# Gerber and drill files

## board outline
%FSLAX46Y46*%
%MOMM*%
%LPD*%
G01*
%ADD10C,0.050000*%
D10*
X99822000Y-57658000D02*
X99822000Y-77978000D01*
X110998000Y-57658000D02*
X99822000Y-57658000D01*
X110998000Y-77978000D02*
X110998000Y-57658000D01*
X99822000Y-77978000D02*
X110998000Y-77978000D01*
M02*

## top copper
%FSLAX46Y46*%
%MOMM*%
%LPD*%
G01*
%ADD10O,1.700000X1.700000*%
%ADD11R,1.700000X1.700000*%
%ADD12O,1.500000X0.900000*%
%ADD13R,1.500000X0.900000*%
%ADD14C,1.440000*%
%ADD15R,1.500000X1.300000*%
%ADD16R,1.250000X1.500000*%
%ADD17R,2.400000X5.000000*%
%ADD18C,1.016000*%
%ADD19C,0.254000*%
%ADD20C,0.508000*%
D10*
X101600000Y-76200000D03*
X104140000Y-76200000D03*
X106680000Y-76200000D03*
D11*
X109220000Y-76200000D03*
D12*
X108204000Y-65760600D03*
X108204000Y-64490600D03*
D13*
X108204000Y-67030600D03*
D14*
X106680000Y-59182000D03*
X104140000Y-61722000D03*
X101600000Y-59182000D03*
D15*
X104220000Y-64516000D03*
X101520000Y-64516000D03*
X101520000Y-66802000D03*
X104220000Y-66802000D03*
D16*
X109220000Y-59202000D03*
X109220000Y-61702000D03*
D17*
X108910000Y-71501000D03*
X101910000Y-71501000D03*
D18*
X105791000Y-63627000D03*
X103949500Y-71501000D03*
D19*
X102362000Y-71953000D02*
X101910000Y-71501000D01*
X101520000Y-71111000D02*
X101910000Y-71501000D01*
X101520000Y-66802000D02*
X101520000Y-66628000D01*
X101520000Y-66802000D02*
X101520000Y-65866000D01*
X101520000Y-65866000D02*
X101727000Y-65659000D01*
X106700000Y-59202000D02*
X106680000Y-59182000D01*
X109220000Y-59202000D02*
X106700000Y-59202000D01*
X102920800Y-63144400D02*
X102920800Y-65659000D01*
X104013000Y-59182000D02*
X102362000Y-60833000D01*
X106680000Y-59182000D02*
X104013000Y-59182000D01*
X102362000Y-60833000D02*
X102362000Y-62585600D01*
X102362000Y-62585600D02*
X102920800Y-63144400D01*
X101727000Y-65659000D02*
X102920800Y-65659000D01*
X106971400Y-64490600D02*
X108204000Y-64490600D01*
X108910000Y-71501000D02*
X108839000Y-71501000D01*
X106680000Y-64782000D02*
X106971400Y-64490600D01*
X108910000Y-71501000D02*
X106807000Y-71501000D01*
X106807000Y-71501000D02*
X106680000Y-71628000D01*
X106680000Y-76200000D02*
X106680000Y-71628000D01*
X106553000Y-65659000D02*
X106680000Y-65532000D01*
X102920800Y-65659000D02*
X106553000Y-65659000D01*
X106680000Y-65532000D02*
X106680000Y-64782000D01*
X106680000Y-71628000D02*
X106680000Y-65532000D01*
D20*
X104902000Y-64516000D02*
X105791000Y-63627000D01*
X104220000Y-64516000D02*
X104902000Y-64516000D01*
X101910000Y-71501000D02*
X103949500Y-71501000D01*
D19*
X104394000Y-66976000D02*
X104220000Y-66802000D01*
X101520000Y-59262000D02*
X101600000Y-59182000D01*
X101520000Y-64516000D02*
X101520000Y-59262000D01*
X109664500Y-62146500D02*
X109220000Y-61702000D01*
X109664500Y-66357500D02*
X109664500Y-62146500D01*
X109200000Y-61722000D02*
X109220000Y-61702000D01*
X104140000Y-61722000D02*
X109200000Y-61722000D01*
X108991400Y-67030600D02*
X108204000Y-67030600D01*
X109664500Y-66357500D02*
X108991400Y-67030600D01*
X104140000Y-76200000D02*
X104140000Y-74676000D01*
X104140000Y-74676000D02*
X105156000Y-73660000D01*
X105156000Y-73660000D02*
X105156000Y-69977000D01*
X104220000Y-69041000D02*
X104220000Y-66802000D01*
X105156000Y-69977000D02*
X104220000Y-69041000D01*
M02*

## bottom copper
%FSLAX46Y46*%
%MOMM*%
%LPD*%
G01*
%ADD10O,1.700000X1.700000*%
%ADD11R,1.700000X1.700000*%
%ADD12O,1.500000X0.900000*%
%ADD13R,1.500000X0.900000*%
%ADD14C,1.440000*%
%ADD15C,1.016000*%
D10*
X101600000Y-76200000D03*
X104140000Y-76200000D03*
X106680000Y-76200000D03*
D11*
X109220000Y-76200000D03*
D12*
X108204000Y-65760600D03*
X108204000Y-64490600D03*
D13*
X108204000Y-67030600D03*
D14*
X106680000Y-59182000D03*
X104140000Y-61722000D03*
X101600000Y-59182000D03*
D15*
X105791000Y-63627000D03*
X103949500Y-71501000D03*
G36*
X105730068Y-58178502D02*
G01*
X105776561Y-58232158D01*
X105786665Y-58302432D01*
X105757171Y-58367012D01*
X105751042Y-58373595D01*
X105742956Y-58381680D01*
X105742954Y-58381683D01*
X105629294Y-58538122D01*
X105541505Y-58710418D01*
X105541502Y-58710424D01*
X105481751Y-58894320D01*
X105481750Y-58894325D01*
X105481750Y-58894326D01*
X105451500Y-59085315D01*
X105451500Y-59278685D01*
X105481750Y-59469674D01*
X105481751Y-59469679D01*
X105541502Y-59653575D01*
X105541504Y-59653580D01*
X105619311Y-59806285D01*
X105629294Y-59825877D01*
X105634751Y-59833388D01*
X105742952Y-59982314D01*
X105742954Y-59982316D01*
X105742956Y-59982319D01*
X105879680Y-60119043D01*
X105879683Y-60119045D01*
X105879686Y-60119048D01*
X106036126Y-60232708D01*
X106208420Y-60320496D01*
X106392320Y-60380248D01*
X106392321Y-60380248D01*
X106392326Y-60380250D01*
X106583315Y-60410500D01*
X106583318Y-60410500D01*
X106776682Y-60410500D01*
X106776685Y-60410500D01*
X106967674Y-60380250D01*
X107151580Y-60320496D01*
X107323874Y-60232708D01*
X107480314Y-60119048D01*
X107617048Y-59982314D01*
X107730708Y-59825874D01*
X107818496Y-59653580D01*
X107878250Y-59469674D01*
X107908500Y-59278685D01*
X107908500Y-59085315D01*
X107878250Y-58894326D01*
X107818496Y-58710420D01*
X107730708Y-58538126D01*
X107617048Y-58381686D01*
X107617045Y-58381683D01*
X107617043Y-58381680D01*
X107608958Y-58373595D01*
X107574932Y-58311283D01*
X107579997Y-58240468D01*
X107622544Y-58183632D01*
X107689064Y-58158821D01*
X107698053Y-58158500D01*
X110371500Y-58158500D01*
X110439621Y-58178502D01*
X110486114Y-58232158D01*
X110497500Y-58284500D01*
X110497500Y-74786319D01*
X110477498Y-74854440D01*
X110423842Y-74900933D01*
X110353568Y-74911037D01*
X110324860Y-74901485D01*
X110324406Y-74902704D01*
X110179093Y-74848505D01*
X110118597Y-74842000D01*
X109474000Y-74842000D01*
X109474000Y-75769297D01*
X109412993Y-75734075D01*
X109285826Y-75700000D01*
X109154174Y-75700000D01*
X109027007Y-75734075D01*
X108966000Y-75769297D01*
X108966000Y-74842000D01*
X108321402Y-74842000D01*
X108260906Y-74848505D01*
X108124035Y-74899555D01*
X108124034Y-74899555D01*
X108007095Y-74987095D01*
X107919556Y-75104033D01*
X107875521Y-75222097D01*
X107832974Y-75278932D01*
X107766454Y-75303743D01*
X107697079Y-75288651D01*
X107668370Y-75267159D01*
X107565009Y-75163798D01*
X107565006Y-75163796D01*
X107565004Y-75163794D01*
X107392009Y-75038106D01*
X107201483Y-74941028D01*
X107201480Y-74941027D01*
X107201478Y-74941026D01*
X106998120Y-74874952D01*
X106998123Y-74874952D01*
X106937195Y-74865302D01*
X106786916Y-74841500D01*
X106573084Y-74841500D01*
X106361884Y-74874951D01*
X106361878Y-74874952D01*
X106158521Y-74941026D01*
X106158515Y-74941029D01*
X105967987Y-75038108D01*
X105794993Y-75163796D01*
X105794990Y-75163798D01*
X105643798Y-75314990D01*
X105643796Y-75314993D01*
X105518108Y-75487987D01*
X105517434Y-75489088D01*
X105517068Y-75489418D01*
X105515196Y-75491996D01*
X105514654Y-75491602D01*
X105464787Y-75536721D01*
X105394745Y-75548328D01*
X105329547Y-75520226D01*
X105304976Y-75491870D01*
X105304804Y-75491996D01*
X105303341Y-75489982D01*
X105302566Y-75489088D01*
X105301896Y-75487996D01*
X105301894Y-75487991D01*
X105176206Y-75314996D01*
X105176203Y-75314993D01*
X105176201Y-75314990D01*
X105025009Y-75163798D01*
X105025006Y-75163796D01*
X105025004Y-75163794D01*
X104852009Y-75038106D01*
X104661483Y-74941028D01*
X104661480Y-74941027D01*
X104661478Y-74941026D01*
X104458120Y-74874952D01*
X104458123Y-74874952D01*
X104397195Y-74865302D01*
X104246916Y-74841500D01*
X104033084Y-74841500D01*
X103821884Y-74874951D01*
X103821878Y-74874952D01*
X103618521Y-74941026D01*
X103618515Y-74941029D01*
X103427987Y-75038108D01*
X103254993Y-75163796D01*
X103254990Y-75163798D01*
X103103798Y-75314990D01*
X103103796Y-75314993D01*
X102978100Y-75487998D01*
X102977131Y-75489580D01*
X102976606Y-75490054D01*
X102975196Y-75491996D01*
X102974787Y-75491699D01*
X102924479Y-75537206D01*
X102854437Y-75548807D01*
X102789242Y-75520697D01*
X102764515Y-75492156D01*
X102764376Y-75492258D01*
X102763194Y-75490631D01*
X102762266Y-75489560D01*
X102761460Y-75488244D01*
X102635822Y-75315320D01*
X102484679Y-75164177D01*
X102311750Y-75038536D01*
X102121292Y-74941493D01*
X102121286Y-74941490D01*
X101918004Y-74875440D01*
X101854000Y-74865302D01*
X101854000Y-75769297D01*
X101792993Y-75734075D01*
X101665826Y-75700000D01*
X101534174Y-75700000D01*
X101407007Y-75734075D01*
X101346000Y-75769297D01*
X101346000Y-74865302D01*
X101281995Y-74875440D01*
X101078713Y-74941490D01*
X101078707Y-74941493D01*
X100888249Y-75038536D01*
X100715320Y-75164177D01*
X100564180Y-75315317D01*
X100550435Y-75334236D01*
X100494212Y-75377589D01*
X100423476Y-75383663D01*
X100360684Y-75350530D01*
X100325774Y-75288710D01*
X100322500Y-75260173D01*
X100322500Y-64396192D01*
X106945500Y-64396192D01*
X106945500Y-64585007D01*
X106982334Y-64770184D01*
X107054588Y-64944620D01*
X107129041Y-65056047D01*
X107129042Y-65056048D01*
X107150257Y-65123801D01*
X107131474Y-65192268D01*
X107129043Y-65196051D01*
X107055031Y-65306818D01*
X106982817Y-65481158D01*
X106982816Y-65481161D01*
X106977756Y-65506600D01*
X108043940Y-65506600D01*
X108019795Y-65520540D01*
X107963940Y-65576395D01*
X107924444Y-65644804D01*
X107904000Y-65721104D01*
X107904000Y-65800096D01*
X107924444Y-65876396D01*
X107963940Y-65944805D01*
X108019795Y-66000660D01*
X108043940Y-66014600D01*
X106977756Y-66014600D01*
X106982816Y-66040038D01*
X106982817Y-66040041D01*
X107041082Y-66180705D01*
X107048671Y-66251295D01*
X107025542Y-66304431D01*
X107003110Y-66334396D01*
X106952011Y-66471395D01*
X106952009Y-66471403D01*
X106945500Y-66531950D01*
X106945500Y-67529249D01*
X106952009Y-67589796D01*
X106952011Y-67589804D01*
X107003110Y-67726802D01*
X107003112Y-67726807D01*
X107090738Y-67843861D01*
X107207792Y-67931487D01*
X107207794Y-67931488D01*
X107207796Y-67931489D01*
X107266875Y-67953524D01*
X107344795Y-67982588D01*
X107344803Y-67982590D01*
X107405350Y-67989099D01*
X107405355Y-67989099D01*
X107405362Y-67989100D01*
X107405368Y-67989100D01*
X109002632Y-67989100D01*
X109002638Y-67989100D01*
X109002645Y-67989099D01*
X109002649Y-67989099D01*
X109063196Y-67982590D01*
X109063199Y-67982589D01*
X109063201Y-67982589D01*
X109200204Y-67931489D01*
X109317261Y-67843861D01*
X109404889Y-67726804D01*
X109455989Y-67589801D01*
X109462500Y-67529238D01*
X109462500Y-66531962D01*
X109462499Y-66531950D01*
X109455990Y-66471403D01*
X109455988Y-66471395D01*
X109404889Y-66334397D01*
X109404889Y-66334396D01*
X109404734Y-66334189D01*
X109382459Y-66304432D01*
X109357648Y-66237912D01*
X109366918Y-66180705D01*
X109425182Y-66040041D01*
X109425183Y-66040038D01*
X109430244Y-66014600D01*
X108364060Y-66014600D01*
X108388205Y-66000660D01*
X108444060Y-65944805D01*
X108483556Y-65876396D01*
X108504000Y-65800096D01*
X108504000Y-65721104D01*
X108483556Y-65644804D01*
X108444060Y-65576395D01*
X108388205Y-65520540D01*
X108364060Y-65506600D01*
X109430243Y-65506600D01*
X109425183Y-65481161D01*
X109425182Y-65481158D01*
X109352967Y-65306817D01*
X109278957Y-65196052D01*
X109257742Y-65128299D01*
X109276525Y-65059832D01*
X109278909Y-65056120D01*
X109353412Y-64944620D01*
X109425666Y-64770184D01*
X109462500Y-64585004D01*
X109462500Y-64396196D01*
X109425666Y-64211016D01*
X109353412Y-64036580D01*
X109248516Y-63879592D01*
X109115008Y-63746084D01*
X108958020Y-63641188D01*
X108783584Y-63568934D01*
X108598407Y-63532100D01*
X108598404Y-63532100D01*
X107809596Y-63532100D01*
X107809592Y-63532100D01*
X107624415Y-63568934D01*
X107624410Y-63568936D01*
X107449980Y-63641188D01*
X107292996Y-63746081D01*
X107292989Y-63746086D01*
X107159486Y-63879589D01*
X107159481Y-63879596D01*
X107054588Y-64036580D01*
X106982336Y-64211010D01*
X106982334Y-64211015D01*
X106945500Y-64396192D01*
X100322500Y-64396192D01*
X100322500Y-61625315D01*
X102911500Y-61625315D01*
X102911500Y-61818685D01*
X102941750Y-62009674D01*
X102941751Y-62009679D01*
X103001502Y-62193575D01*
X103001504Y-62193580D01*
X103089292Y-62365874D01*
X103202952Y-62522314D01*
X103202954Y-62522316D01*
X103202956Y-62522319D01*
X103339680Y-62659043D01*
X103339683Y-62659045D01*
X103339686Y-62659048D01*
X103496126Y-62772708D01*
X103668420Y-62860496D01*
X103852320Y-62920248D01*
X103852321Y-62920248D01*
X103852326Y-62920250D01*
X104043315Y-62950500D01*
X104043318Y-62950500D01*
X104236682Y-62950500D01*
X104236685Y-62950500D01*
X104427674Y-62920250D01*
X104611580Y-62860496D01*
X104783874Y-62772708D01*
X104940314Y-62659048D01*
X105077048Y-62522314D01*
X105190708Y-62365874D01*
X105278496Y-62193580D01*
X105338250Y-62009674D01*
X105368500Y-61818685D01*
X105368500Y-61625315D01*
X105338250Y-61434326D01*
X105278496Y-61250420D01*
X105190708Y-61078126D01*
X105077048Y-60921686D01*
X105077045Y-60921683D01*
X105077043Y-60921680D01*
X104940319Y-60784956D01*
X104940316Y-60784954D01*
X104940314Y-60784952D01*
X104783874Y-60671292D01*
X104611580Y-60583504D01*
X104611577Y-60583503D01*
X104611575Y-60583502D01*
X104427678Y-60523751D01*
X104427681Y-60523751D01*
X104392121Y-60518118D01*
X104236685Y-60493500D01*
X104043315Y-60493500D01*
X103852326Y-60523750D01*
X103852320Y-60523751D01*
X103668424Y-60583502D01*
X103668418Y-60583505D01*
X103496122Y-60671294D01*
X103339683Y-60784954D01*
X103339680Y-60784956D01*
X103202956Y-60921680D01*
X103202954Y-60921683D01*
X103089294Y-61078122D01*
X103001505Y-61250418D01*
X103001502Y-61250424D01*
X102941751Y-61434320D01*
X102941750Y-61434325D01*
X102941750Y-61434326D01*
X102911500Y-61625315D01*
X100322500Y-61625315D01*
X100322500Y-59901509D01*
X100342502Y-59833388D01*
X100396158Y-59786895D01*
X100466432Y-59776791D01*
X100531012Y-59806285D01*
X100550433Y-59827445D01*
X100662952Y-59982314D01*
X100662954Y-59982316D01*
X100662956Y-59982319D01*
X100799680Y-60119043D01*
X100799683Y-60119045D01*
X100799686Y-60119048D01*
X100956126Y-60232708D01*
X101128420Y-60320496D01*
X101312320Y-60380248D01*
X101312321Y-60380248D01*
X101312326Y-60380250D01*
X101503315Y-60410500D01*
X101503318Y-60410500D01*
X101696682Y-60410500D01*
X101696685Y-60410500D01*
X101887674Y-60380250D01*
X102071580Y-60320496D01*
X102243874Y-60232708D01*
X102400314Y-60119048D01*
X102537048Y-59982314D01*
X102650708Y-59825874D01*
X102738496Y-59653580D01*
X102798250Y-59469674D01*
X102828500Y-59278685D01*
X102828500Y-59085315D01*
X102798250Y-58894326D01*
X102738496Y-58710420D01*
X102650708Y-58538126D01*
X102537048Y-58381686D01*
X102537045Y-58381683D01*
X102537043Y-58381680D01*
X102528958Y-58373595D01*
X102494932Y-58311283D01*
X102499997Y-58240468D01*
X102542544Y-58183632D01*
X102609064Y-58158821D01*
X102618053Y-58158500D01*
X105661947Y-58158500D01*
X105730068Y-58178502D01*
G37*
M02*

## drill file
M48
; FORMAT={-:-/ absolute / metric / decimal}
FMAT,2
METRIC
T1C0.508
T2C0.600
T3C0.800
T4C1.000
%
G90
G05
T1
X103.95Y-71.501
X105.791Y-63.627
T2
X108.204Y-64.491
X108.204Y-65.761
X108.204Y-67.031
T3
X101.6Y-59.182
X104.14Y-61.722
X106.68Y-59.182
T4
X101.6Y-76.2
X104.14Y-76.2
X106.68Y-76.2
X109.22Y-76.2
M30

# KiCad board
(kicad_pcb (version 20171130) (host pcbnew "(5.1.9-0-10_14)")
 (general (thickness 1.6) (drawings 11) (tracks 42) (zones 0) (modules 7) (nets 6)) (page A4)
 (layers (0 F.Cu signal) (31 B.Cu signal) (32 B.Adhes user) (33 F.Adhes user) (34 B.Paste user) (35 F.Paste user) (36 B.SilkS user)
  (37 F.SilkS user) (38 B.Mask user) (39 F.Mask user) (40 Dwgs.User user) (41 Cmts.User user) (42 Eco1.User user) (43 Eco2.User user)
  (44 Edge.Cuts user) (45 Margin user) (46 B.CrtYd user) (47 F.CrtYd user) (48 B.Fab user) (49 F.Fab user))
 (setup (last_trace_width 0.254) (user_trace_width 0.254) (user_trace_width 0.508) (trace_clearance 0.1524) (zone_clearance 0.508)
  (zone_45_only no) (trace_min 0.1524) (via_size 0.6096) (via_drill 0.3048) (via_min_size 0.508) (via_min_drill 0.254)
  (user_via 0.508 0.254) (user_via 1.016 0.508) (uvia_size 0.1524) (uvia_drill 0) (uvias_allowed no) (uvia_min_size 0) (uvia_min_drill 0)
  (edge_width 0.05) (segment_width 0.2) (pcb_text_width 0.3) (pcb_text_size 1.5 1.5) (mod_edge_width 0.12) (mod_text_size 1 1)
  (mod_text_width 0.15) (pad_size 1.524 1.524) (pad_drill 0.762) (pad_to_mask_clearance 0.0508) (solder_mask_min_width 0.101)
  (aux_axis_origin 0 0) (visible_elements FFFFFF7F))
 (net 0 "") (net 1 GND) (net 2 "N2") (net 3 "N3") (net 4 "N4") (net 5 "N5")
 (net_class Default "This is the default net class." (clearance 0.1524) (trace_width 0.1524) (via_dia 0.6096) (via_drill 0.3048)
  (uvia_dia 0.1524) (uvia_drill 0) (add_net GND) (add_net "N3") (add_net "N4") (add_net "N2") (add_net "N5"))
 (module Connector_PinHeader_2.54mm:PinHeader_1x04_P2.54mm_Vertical (layer B.Cu) (at 109.22 76.2 90)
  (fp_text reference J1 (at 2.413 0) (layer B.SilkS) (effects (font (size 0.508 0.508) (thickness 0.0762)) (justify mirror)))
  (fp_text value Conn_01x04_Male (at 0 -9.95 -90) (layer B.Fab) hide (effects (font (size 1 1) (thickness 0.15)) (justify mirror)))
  (pad 4 thru_hole oval (at 0 -7.62 90) (size 1.7 1.7) (drill 1) (layers *.Cu *.Mask) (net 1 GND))
  (pad 3 thru_hole oval (at 0 -5.08 90) (size 1.7 1.7) (drill 1) (layers *.Cu *.Mask) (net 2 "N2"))
  (pad 2 thru_hole oval (at 0 -2.54 90) (size 1.7 1.7) (drill 1) (layers *.Cu *.Mask) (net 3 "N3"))
  (pad 1 thru_hole rect (at 0 0 90) (size 1.7 1.7) (drill 1) (layers *.Cu *.Mask) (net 1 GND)))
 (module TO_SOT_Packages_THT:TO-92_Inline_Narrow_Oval (layer F.Cu) (at 108.204 67.0306 90)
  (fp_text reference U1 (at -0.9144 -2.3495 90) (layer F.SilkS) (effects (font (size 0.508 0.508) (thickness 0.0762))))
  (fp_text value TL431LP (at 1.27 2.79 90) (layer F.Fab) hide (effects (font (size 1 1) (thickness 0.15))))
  (pad 2 thru_hole oval (at 1.27 0 270) (size 0.9 1.5) (drill 0.6) (layers *.Cu *.Mask) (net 1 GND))
  (pad 3 thru_hole oval (at 2.54 0 270) (size 0.9 1.5) (drill 0.6) (layers *.Cu *.Mask) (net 3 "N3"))
  (pad 1 thru_hole rect (at 0 0 270) (size 0.9 1.5) (drill 0.6) (layers *.Cu *.Mask) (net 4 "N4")))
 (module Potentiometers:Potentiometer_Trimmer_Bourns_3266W (layer F.Cu) (at 106.68 59.182)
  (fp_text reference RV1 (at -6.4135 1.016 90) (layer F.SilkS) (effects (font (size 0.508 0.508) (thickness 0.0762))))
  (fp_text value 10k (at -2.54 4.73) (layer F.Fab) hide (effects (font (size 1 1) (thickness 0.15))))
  (pad 1 thru_hole circle (at 0 0) (size 1.44 1.44) (drill 0.8) (layers *.Cu *.Mask) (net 3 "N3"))
  (pad 2 thru_hole circle (at -2.54 2.54) (size 1.44 1.44) (drill 0.8) (layers *.Cu *.Mask) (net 4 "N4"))
  (pad 3 thru_hole circle (at -5.08 0) (size 1.44 1.44) (drill 0.8) (layers *.Cu *.Mask) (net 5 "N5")))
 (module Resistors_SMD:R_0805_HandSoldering (layer F.Cu) (at 102.87 64.516 180)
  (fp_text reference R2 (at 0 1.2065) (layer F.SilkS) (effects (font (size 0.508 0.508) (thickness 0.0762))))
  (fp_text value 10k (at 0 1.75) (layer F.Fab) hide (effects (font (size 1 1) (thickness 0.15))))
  (pad 1 smd rect (at -1.35 0 180) (size 1.5 1.3) (layers F.Cu F.Paste F.Mask) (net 1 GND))
  (pad 2 smd rect (at 1.35 0 180) (size 1.5 1.3) (layers F.Cu F.Paste F.Mask) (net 5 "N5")))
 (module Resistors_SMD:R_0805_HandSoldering (layer F.Cu) (at 102.87 66.802)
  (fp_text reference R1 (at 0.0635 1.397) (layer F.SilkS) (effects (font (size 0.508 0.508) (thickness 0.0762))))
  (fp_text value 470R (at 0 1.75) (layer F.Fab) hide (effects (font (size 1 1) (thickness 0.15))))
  (pad 1 smd rect (at -1.35 0) (size 1.5 1.3) (layers F.Cu F.Paste F.Mask) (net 3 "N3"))
  (pad 2 smd rect (at 1.35 0) (size 1.5 1.3) (layers F.Cu F.Paste F.Mask) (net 2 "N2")))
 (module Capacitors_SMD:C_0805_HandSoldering (layer F.Cu) (at 109.22 60.452 270)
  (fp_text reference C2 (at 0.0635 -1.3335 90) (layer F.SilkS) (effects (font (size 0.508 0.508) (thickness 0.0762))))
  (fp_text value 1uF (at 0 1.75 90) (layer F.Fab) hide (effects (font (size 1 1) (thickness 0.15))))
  (pad 1 smd rect (at -1.25 0 270) (size 1.5 1.25) (layers F.Cu F.Paste F.Mask) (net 3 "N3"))
  (pad 2 smd rect (at 1.25 0 270) (size 1.5 1.25) (layers F.Cu F.Paste F.Mask) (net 4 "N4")))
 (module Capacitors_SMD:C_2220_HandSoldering (layer F.Cu) (at 105.41 71.501 180)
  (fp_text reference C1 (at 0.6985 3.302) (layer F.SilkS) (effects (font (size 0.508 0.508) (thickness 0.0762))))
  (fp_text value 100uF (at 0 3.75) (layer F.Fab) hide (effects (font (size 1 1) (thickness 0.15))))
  (pad 1 smd rect (at -3.5 0 180) (size 2.4 5) (layers F.Cu F.Paste F.Mask) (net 3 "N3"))
  (pad 2 smd rect (at 3.5 0 180) (size 2.4 5) (layers F.Cu F.Paste F.Mask) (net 1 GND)))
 (gr_line (start 99.822 57.658) (end 99.822 77.978) (layer Edge.Cuts) (width 0.05))
 (gr_line (start 110.998 57.658) (end 99.822 57.658) (layer Edge.Cuts) (width 0.05))
 (gr_line (start 110.998 77.978) (end 110.998 57.658) (layer Edge.Cuts) (width 0.05))
 (gr_line (start 99.822 77.978) (end 110.998 77.978) (layer Edge.Cuts) (width 0.05))
 (segment (start 102.362 71.953) (end 101.91 71.501) (width 0.254) (layer F.Cu) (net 1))
 (segment (start 101.52 71.111) (end 101.91 71.501) (width 0.254) (layer F.Cu) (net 1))
 (segment (start 101.52 66.802) (end 101.52 66.628) (width 0.254) (layer F.Cu) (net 3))
 (segment (start 101.52 66.802) (end 101.52 65.866) (width 0.254) (layer F.Cu) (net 3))
 (segment (start 101.52 65.866) (end 101.727 65.659) (width 0.254) (layer F.Cu) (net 3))
 (segment (start 106.7 59.202) (end 106.68 59.182) (width 0.254) (layer F.Cu) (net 3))
 (segment (start 109.22 59.202) (end 106.7 59.202) (width 0.254) (layer F.Cu) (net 3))
 (segment (start 102.9208 63.1444) (end 102.9208 65.659) (width 0.254) (layer F.Cu) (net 3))
 (segment (start 104.013 59.182) (end 102.362 60.833) (width 0.254) (layer F.Cu) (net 3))
 (segment (start 106.68 59.182) (end 104.013 59.182) (width 0.254) (layer F.Cu) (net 3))
 (segment (start 102.362 60.833) (end 102.362 62.5856) (width 0.254) (layer F.Cu) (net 3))
 (segment (start 102.362 62.5856) (end 102.9208 63.1444) (width 0.254) (layer F.Cu) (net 3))
 (segment (start 101.727 65.659) (end 102.9208 65.659) (width 0.254) (layer F.Cu) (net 3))
 (segment (start 106.9714 64.4906) (end 108.204 64.4906) (width 0.254) (layer F.Cu) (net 3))
 (segment (start 108.91 71.501) (end 108.839 71.501) (width 0.254) (layer F.Cu) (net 3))
 (segment (start 106.68 64.782) (end 106.9714 64.4906) (width 0.254) (layer F.Cu) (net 3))
 (segment (start 108.91 71.501) (end 106.807 71.501) (width 0.254) (layer F.Cu) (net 3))
 (segment (start 106.807 71.501) (end 106.68 71.628) (width 0.254) (layer F.Cu) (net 3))
 (segment (start 106.68 76.2) (end 106.68 71.628) (width 0.254) (layer F.Cu) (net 3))
 (segment (start 106.553 65.659) (end 106.68 65.532) (width 0.254) (layer F.Cu) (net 3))
 (segment (start 102.9208 65.659) (end 106.553 65.659) (width 0.254) (layer F.Cu) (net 3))
 (segment (start 106.68 65.532) (end 106.68 64.782) (width 0.254) (layer F.Cu) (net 3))
 (segment (start 106.68 71.628) (end 106.68 65.532) (width 0.254) (layer F.Cu) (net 3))
 (segment (start 104.902 64.516) (end 105.791 63.627) (width 0.508) (layer F.Cu) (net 1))
 (via (at 105.791 63.627) (size 1.016) (drill 0.508) (layers F.Cu B.Cu) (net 1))
 (segment (start 104.22 64.516) (end 104.902 64.516) (width 0.508) (layer F.Cu) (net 1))
 (via (at 103.9495 71.501) (size 1.016) (drill 0.508) (layers F.Cu B.Cu) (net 1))
 (segment (start 101.91 71.501) (end 103.9495 71.501) (width 0.508) (layer F.Cu) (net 1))
 (segment (start 104.394 66.976) (end 104.22 66.802) (width 0.254) (layer F.Cu) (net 2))
 (segment (start 101.52 59.262) (end 101.6 59.182) (width 0.254) (layer F.Cu) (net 5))
 (segment (start 101.52 64.516) (end 101.52 59.262) (width 0.254) (layer F.Cu) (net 5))
 (segment (start 109.6645 62.1465) (end 109.22 61.702) (width 0.254) (layer F.Cu) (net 4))
 (segment (start 109.6645 66.3575) (end 109.6645 62.1465) (width 0.254) (layer F.Cu) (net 4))
 (segment (start 109.2 61.722) (end 109.22 61.702) (width 0.254) (layer F.Cu) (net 4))
 (segment (start 104.14 61.722) (end 109.2 61.722) (width 0.254) (layer F.Cu) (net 4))
 (segment (start 108.9914 67.0306) (end 108.204 67.0306) (width 0.254) (layer F.Cu) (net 4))
 (segment (start 109.6645 66.3575) (end 108.9914 67.0306) (width 0.254) (layer F.Cu) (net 4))
 (segment (start 104.14 76.2) (end 104.14 74.676) (width 0.254) (layer F.Cu) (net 2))
 (segment (start 104.14 74.676) (end 105.156 73.66) (width 0.254) (layer F.Cu) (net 2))
 (segment (start 105.156 73.66) (end 105.156 69.977) (width 0.254) (layer F.Cu) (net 2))
 (segment (start 104.22 69.041) (end 104.22 66.802) (width 0.254) (layer F.Cu) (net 2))
 (segment (start 105.156 69.977) (end 104.22 69.041) (width 0.254) (layer F.Cu) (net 2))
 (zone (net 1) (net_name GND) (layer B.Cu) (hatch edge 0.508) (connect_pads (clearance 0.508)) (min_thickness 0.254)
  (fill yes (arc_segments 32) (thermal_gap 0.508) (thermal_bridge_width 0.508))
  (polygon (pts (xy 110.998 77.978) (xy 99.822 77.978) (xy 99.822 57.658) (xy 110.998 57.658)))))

